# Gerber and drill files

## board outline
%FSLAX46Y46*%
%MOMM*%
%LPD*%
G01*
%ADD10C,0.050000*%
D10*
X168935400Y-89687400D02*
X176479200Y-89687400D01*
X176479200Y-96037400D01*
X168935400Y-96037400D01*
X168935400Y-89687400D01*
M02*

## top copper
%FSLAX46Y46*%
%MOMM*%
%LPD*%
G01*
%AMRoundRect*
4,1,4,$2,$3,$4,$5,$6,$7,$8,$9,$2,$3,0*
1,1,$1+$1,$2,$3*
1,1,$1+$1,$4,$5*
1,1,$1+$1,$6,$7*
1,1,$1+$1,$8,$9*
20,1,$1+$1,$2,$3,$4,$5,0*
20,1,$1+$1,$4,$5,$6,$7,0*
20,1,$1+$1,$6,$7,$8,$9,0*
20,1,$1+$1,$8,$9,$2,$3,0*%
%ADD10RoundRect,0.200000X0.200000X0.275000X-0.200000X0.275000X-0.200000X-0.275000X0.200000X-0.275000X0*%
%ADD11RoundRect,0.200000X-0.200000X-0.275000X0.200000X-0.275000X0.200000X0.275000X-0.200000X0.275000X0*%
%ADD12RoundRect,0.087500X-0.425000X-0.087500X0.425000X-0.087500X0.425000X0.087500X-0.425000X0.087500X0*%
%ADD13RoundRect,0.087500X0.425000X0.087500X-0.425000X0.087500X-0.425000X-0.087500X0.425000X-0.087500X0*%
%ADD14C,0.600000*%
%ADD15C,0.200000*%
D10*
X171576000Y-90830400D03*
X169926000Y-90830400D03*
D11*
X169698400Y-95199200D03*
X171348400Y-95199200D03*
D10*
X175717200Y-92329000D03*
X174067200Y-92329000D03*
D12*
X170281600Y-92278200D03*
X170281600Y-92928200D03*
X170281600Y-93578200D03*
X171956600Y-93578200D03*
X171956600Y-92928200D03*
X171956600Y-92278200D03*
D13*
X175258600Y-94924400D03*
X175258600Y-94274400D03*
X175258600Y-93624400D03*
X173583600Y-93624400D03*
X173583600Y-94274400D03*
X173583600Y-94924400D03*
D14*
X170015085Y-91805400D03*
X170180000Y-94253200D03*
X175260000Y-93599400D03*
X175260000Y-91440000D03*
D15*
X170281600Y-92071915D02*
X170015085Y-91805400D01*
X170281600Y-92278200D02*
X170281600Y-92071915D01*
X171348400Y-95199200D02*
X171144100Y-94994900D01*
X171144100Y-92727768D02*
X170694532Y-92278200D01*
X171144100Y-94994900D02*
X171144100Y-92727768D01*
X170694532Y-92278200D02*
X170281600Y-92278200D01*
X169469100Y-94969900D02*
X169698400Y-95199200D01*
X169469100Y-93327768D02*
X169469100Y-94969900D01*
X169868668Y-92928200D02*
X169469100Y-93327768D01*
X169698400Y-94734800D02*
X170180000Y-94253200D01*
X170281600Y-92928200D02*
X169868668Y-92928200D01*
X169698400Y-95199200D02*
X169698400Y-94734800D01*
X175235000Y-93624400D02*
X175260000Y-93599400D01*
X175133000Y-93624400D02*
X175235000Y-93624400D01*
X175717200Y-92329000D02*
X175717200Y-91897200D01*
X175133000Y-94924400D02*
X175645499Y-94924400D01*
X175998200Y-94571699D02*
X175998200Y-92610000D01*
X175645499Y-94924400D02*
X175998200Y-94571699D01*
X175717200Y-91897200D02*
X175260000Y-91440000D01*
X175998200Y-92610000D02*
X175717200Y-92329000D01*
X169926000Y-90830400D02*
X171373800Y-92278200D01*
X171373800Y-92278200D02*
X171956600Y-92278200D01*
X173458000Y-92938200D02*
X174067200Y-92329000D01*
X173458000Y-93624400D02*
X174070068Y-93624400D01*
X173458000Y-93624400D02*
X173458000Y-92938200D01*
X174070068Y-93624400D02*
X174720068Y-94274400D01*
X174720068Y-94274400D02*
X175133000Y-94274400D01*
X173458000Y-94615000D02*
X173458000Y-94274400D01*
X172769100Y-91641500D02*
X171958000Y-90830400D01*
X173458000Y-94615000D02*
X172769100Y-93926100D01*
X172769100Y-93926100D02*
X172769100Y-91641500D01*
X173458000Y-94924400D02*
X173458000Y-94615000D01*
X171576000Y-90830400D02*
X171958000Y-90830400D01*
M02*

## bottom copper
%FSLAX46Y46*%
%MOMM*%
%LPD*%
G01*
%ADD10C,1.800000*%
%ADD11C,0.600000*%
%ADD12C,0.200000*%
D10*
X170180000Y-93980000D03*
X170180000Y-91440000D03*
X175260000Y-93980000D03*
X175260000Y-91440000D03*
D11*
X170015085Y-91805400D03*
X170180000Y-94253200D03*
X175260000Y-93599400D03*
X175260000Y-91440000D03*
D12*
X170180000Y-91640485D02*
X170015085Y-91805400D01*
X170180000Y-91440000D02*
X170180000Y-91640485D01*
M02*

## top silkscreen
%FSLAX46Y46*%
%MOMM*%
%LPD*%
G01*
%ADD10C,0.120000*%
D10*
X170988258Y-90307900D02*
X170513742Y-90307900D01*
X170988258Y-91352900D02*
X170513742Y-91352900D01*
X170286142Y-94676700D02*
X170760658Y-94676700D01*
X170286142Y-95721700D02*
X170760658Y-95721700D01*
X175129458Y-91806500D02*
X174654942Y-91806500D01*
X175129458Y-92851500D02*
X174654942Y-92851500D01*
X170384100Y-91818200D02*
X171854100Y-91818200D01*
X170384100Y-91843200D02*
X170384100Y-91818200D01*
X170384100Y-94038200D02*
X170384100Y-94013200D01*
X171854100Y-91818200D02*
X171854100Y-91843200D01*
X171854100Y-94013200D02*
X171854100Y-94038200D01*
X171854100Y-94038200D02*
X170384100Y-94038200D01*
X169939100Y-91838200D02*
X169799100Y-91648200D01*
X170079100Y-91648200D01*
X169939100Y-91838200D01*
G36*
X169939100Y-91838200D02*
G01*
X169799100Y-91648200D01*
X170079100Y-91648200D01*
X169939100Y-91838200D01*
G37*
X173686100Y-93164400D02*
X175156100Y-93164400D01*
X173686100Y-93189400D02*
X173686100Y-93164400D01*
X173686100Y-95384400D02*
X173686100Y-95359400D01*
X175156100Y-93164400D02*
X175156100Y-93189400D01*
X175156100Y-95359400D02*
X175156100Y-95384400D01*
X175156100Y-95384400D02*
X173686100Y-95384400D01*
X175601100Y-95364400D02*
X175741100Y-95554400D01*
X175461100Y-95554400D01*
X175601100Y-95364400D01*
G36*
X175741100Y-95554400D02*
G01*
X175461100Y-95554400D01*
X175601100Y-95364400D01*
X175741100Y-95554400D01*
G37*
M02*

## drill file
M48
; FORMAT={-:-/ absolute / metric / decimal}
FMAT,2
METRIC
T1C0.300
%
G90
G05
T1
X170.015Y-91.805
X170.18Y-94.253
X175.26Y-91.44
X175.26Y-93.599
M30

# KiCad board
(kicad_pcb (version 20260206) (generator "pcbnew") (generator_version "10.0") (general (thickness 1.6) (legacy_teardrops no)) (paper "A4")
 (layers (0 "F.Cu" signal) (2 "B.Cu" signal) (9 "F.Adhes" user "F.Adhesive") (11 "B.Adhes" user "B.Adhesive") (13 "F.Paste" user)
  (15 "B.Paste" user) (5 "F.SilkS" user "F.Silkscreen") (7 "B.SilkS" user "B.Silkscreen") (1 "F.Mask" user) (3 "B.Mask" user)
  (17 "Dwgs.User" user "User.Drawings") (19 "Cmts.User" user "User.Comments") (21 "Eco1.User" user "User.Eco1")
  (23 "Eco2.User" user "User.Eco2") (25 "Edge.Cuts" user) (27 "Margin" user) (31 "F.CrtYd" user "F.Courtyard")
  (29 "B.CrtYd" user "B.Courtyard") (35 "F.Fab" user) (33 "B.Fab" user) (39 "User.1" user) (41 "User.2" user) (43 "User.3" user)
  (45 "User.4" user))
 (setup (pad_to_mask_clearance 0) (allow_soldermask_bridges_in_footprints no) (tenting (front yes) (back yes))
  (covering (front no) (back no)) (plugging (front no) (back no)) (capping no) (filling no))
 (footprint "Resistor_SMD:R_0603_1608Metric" (layer "F.Cu") (at 170.751 90.8304 180)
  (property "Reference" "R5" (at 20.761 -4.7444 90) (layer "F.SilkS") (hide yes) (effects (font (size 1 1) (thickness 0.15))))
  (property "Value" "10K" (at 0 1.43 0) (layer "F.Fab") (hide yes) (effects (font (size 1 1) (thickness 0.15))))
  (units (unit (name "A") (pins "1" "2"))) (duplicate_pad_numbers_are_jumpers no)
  (fp_line (start -0.237258 0.5225) (end 0.237258 0.5225) (stroke (width 0.12) (type solid)) (layer "F.SilkS"))
  (fp_line (start -0.237258 -0.5225) (end 0.237258 -0.5225) (stroke (width 0.12) (type solid)) (layer "F.SilkS"))
  (pad "1" smd roundrect (at -0.825 0 180) (size 0.8 0.95) (layers "F.Cu" "F.Mask" "F.Paste") (roundrect_rratio 0.25) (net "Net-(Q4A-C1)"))
  (pad "2" smd roundrect (at 0.825 0 180) (size 0.8 0.95) (layers "F.Cu" "F.Mask" "F.Paste") (roundrect_rratio 0.25) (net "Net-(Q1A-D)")))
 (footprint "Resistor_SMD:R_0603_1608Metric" (layer "F.Cu") (at 170.5234 95.1992)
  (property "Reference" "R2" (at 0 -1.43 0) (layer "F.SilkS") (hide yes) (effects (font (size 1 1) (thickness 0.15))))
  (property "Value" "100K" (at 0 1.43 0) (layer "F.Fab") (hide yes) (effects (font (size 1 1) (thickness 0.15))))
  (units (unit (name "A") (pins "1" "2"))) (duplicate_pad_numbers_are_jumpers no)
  (fp_line (start -0.237258 -0.5225) (end 0.237258 -0.5225) (stroke (width 0.12) (type solid)) (layer "F.SilkS"))
  (fp_line (start -0.237258 0.5225) (end 0.237258 0.5225) (stroke (width 0.12) (type solid)) (layer "F.SilkS"))
  (pad "1" smd roundrect (at -0.825 0) (size 0.8 0.95) (layers "F.Cu" "F.Mask" "F.Paste") (roundrect_rratio 0.25) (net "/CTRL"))
  (pad "2" smd roundrect (at 0.825 0) (size 0.8 0.95) (layers "F.Cu" "F.Mask" "F.Paste") (roundrect_rratio 0.25) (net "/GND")))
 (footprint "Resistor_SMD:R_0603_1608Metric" (layer "F.Cu") (at 174.8922 92.329 180)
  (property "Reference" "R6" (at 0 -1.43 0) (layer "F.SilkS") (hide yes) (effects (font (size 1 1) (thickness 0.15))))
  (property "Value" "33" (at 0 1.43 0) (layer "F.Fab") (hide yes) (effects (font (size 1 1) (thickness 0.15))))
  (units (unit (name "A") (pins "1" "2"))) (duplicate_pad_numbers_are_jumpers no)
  (fp_line (start -0.237258 0.5225) (end 0.237258 0.5225) (stroke (width 0.12) (type solid)) (layer "F.SilkS"))
  (fp_line (start -0.237258 -0.5225) (end 0.237258 -0.5225) (stroke (width 0.12) (type solid)) (layer "F.SilkS"))
  (pad "1" smd roundrect (at -0.825 0 180) (size 0.8 0.95) (layers "F.Cu" "F.Mask" "F.Paste") (roundrect_rratio 0.25) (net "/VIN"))
  (pad "2" smd roundrect (at 0.825 0 180) (size 0.8 0.95) (layers "F.Cu" "F.Mask" "F.Paste") (roundrect_rratio 0.25) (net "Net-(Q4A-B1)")))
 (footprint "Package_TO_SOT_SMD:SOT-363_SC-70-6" (layer "F.Cu") (at 171.1191 92.9282)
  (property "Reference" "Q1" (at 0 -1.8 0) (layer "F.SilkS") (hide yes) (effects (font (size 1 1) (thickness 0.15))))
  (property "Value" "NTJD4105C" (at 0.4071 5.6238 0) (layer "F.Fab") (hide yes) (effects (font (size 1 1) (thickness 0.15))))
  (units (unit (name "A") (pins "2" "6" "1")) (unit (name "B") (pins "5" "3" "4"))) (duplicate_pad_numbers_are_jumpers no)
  (fp_line (start -0.735 -1.11) (end 0.735 -1.11) (stroke (width 0.12) (type solid)) (layer "F.SilkS"))
  (fp_line (start -0.735 -1.085) (end -0.735 -1.11) (stroke (width 0.12) (type solid)) (layer "F.SilkS"))
  (fp_line (start -0.735 1.11) (end -0.735 1.085) (stroke (width 0.12) (type solid)) (layer "F.SilkS"))
  (fp_line (start 0.735 -1.11) (end 0.735 -1.085) (stroke (width 0.12) (type solid)) (layer "F.SilkS"))
  (fp_line (start 0.735 1.085) (end 0.735 1.11) (stroke (width 0.12) (type solid)) (layer "F.SilkS"))
  (fp_line (start 0.735 1.11) (end -0.735 1.11) (stroke (width 0.12) (type solid)) (layer "F.SilkS"))
  (fp_poly (pts (xy -1.18 -1.09) (xy -1.32 -1.28) (xy -1.04 -1.28)) (stroke (width 0.12) (type solid)) (fill yes) (layer "F.SilkS"))
  (pad "1" smd roundrect (at -0.8375 -0.65) (size 1.025 0.35) (layers "F.Cu" "F.Mask" "F.Paste") (roundrect_rratio 0.25) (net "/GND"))
  (pad "2" smd roundrect (at -0.8375 0) (size 1.025 0.35) (layers "F.Cu" "F.Mask" "F.Paste") (roundrect_rratio 0.25) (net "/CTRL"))
  (pad "3" smd roundrect (at -0.8375 0.65) (size 1.025 0.35) (layers "F.Cu" "F.Mask" "F.Paste") (roundrect_rratio 0.25))
  (pad "4" smd roundrect (at 0.8375 0.65) (size 1.025 0.35) (layers "F.Cu" "F.Mask" "F.Paste") (roundrect_rratio 0.25))
  (pad "5" smd roundrect (at 0.8375 0) (size 1.025 0.35) (layers "F.Cu" "F.Mask" "F.Paste") (roundrect_rratio 0.25))
  (pad "6" smd roundrect (at 0.8375 -0.65) (size 1.025 0.35) (layers "F.Cu" "F.Mask" "F.Paste") (roundrect_rratio 0.25) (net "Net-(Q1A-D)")))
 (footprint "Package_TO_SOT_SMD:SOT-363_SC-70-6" (layer "F.Cu") (at 174.4211 94.2744 180)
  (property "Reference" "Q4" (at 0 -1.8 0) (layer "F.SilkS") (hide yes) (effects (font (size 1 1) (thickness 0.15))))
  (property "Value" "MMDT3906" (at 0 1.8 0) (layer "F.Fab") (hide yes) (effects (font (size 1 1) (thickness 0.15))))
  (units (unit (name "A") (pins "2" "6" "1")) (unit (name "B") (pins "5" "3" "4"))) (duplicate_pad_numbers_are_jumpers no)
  (fp_line (start 0.735 1.11) (end -0.735 1.11) (stroke (width 0.12) (type solid)) (layer "F.SilkS"))
  (fp_line (start 0.735 1.085) (end 0.735 1.11) (stroke (width 0.12) (type solid)) (layer "F.SilkS"))
  (fp_line (start 0.735 -1.11) (end 0.735 -1.085) (stroke (width 0.12) (type solid)) (layer "F.SilkS"))
  (fp_line (start -0.735 1.11) (end -0.735 1.085) (stroke (width 0.12) (type solid)) (layer "F.SilkS"))
  (fp_line (start -0.735 -1.085) (end -0.735 -1.11) (stroke (width 0.12) (type solid)) (layer "F.SilkS"))
  (fp_line (start -0.735 -1.11) (end 0.735 -1.11) (stroke (width 0.12) (type solid)) (layer "F.SilkS"))
  (fp_poly (pts (xy -1.18 -1.09) (xy -1.32 -1.28) (xy -1.04 -1.28)) (stroke (width 0.12) (type solid)) (fill yes) (layer "F.SilkS"))
  (pad "1" smd roundrect (at -0.8375 -0.65 180) (size 1.025 0.35) (layers "F.Cu" "F.Mask" "F.Paste") (roundrect_rratio 0.25) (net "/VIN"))
  (pad "2" smd roundrect (at -0.8375 0 180) (size 1.025 0.35) (layers "F.Cu" "F.Mask" "F.Paste") (roundrect_rratio 0.25)
   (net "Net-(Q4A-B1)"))
  (pad "3" smd roundrect (at -0.8375 0.65 180) (size 1.025 0.35) (layers "F.Cu" "F.Mask" "F.Paste") (roundrect_rratio 0.25) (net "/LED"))
  (pad "4" smd roundrect (at 0.8375 0.65 180) (size 1.025 0.35) (layers "F.Cu" "F.Mask" "F.Paste") (roundrect_rratio 0.25)
   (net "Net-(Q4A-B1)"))
  (pad "5" smd roundrect (at 0.8375 0 180) (size 1.025 0.35) (layers "F.Cu" "F.Mask" "F.Paste") (roundrect_rratio 0.25) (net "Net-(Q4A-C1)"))
  (pad "6" smd roundrect (at 0.8375 -0.65 180) (size 1.025 0.35) (layers "F.Cu" "F.Mask" "F.Paste") (roundrect_rratio 0.25)
   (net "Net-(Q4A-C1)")))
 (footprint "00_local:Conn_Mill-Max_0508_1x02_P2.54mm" (layer "B.Cu") (at 170.18 93.98 90)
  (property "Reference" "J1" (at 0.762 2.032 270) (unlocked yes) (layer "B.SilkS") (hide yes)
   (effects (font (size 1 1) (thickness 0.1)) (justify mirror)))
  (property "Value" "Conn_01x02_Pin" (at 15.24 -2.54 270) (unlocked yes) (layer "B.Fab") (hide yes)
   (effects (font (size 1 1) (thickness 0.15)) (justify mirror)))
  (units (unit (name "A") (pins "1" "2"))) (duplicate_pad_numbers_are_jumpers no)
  (pad "1" smd circle (at 0 0 90) (size 1.8 1.8) (layers "B.Cu" "B.Mask" "B.Paste") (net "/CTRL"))
  (pad "2" smd circle (at 2.54 0 90) (size 1.8 1.8) (layers "B.Cu" "B.Mask" "B.Paste") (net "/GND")))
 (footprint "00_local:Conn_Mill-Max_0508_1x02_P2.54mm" (layer "B.Cu") (at 175.26 93.98 90)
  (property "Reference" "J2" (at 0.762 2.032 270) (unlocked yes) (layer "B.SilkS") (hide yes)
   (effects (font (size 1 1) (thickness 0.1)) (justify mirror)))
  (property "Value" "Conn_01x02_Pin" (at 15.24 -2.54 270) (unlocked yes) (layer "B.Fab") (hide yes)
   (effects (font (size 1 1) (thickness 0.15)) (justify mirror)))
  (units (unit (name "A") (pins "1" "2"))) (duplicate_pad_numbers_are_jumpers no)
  (pad "1" smd circle (at 0 0 90) (size 1.8 1.8) (layers "B.Cu" "B.Mask" "B.Paste") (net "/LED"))
  (pad "2" smd circle (at 2.54 0 90) (size 1.8 1.8) (layers "B.Cu" "B.Mask" "B.Paste") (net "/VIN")))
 (gr_rect (start 168.9354 89.6874) (end 176.4792 96.0374) (stroke (width 0.05) (type default)) (fill no) (layer "Edge.Cuts"))
 (segment (start 170.2816 92.071915) (end 170.015085 91.8054) (width 0.2) (layer "F.Cu") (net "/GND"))
 (segment (start 170.2816 92.2782) (end 170.2816 92.071915) (width 0.2) (layer "F.Cu") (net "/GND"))
 (segment (start 171.3484 95.1992) (end 171.1441 94.9949) (width 0.2) (layer "F.Cu") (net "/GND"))
 (segment (start 171.1441 92.727768) (end 170.694532 92.2782) (width 0.2) (layer "F.Cu") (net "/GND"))
 (segment (start 171.1441 94.9949) (end 171.1441 92.727768) (width 0.2) (layer "F.Cu") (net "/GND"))
 (segment (start 170.694532 92.2782) (end 170.2816 92.2782) (width 0.2) (layer "F.Cu") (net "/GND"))
 (via (at 170.015085 91.8054) (size 0.6) (drill 0.3) (layers "F.Cu" "B.Cu") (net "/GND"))
 (segment (start 170.18 91.640485) (end 170.015085 91.8054) (width 0.2) (layer "B.Cu") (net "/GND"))
 (segment (start 170.18 91.44) (end 170.18 91.640485) (width 0.2) (layer "B.Cu") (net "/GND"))
 (segment (start 169.4691 94.9699) (end 169.6984 95.1992) (width 0.2) (layer "F.Cu") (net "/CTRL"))
 (segment (start 169.4691 93.327768) (end 169.4691 94.9699) (width 0.2) (layer "F.Cu") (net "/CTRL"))
 (segment (start 169.868668 92.9282) (end 169.4691 93.327768) (width 0.2) (layer "F.Cu") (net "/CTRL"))
 (segment (start 169.6984 94.7348) (end 170.18 94.2532) (width 0.2) (layer "F.Cu") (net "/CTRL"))
 (segment (start 170.2816 92.9282) (end 169.868668 92.9282) (width 0.2) (layer "F.Cu") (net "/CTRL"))
 (segment (start 169.6984 95.1992) (end 169.6984 94.7348) (width 0.2) (layer "F.Cu") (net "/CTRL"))
 (via (at 170.18 94.2532) (size 0.6) (drill 0.3) (layers "F.Cu" "B.Cu") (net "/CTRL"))
 (segment (start 175.235 93.6244) (end 175.26 93.5994) (width 0.2) (layer "F.Cu") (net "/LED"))
 (segment (start 175.133 93.6244) (end 175.235 93.6244) (width 0.2) (layer "F.Cu") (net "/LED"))
 (via (at 175.26 93.5994) (size 0.6) (drill 0.3) (layers "F.Cu" "B.Cu") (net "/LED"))
 (segment (start 175.7172 92.329) (end 175.7172 91.8972) (width 0.2) (layer "F.Cu") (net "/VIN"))
 (segment (start 175.133 94.9244) (end 175.645499 94.9244) (width 0.2) (layer "F.Cu") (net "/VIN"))
 (segment (start 175.9982 94.571699) (end 175.9982 92.61) (width 0.2) (layer "F.Cu") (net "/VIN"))
 (segment (start 175.645499 94.9244) (end 175.9982 94.571699) (width 0.2) (layer "F.Cu") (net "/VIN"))
 (segment (start 175.7172 91.8972) (end 175.26 91.44) (width 0.2) (layer "F.Cu") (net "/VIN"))
 (segment (start 175.9982 92.61) (end 175.7172 92.329) (width 0.2) (layer "F.Cu") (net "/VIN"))
 (via (at 175.26 91.44) (size 0.6) (drill 0.3) (layers "F.Cu" "B.Cu") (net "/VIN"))
 (segment (start 169.926 90.8304) (end 171.3738 92.2782) (width 0.2) (layer "F.Cu") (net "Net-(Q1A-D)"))
 (segment (start 171.3738 92.2782) (end 171.9566 92.2782) (width 0.2) (layer "F.Cu") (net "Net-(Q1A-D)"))
 (segment (start 173.458 92.9382) (end 174.0672 92.329) (width 0.2) (layer "F.Cu") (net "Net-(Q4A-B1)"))
 (segment (start 173.458 93.6244) (end 174.070068 93.6244) (width 0.2) (layer "F.Cu") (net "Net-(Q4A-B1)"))
 (segment (start 173.458 93.6244) (end 173.458 92.9382) (width 0.2) (layer "F.Cu") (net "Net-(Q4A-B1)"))
 (segment (start 174.070068 93.6244) (end 174.720068 94.2744) (width 0.2) (layer "F.Cu") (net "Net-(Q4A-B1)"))
 (segment (start 174.720068 94.2744) (end 175.133 94.2744) (width 0.2) (layer "F.Cu") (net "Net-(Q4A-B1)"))
 (segment (start 173.458 94.615) (end 173.458 94.2744) (width 0.2) (layer "F.Cu") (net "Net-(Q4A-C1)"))
 (segment (start 172.7691 91.6415) (end 171.958 90.8304) (width 0.2) (layer "F.Cu") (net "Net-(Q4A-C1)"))
 (segment (start 173.458 94.615) (end 172.7691 93.9261) (width 0.2) (layer "F.Cu") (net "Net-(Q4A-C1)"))
 (segment (start 172.7691 93.9261) (end 172.7691 91.6415) (width 0.2) (layer "F.Cu") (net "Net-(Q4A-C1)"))
 (segment (start 173.458 94.9244) (end 173.458 94.615) (width 0.2) (layer "F.Cu") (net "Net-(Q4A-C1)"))
 (segment (start 171.576 90.8304) (end 171.958 90.8304) (width 0.2) (layer "F.Cu") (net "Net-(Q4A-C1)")))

